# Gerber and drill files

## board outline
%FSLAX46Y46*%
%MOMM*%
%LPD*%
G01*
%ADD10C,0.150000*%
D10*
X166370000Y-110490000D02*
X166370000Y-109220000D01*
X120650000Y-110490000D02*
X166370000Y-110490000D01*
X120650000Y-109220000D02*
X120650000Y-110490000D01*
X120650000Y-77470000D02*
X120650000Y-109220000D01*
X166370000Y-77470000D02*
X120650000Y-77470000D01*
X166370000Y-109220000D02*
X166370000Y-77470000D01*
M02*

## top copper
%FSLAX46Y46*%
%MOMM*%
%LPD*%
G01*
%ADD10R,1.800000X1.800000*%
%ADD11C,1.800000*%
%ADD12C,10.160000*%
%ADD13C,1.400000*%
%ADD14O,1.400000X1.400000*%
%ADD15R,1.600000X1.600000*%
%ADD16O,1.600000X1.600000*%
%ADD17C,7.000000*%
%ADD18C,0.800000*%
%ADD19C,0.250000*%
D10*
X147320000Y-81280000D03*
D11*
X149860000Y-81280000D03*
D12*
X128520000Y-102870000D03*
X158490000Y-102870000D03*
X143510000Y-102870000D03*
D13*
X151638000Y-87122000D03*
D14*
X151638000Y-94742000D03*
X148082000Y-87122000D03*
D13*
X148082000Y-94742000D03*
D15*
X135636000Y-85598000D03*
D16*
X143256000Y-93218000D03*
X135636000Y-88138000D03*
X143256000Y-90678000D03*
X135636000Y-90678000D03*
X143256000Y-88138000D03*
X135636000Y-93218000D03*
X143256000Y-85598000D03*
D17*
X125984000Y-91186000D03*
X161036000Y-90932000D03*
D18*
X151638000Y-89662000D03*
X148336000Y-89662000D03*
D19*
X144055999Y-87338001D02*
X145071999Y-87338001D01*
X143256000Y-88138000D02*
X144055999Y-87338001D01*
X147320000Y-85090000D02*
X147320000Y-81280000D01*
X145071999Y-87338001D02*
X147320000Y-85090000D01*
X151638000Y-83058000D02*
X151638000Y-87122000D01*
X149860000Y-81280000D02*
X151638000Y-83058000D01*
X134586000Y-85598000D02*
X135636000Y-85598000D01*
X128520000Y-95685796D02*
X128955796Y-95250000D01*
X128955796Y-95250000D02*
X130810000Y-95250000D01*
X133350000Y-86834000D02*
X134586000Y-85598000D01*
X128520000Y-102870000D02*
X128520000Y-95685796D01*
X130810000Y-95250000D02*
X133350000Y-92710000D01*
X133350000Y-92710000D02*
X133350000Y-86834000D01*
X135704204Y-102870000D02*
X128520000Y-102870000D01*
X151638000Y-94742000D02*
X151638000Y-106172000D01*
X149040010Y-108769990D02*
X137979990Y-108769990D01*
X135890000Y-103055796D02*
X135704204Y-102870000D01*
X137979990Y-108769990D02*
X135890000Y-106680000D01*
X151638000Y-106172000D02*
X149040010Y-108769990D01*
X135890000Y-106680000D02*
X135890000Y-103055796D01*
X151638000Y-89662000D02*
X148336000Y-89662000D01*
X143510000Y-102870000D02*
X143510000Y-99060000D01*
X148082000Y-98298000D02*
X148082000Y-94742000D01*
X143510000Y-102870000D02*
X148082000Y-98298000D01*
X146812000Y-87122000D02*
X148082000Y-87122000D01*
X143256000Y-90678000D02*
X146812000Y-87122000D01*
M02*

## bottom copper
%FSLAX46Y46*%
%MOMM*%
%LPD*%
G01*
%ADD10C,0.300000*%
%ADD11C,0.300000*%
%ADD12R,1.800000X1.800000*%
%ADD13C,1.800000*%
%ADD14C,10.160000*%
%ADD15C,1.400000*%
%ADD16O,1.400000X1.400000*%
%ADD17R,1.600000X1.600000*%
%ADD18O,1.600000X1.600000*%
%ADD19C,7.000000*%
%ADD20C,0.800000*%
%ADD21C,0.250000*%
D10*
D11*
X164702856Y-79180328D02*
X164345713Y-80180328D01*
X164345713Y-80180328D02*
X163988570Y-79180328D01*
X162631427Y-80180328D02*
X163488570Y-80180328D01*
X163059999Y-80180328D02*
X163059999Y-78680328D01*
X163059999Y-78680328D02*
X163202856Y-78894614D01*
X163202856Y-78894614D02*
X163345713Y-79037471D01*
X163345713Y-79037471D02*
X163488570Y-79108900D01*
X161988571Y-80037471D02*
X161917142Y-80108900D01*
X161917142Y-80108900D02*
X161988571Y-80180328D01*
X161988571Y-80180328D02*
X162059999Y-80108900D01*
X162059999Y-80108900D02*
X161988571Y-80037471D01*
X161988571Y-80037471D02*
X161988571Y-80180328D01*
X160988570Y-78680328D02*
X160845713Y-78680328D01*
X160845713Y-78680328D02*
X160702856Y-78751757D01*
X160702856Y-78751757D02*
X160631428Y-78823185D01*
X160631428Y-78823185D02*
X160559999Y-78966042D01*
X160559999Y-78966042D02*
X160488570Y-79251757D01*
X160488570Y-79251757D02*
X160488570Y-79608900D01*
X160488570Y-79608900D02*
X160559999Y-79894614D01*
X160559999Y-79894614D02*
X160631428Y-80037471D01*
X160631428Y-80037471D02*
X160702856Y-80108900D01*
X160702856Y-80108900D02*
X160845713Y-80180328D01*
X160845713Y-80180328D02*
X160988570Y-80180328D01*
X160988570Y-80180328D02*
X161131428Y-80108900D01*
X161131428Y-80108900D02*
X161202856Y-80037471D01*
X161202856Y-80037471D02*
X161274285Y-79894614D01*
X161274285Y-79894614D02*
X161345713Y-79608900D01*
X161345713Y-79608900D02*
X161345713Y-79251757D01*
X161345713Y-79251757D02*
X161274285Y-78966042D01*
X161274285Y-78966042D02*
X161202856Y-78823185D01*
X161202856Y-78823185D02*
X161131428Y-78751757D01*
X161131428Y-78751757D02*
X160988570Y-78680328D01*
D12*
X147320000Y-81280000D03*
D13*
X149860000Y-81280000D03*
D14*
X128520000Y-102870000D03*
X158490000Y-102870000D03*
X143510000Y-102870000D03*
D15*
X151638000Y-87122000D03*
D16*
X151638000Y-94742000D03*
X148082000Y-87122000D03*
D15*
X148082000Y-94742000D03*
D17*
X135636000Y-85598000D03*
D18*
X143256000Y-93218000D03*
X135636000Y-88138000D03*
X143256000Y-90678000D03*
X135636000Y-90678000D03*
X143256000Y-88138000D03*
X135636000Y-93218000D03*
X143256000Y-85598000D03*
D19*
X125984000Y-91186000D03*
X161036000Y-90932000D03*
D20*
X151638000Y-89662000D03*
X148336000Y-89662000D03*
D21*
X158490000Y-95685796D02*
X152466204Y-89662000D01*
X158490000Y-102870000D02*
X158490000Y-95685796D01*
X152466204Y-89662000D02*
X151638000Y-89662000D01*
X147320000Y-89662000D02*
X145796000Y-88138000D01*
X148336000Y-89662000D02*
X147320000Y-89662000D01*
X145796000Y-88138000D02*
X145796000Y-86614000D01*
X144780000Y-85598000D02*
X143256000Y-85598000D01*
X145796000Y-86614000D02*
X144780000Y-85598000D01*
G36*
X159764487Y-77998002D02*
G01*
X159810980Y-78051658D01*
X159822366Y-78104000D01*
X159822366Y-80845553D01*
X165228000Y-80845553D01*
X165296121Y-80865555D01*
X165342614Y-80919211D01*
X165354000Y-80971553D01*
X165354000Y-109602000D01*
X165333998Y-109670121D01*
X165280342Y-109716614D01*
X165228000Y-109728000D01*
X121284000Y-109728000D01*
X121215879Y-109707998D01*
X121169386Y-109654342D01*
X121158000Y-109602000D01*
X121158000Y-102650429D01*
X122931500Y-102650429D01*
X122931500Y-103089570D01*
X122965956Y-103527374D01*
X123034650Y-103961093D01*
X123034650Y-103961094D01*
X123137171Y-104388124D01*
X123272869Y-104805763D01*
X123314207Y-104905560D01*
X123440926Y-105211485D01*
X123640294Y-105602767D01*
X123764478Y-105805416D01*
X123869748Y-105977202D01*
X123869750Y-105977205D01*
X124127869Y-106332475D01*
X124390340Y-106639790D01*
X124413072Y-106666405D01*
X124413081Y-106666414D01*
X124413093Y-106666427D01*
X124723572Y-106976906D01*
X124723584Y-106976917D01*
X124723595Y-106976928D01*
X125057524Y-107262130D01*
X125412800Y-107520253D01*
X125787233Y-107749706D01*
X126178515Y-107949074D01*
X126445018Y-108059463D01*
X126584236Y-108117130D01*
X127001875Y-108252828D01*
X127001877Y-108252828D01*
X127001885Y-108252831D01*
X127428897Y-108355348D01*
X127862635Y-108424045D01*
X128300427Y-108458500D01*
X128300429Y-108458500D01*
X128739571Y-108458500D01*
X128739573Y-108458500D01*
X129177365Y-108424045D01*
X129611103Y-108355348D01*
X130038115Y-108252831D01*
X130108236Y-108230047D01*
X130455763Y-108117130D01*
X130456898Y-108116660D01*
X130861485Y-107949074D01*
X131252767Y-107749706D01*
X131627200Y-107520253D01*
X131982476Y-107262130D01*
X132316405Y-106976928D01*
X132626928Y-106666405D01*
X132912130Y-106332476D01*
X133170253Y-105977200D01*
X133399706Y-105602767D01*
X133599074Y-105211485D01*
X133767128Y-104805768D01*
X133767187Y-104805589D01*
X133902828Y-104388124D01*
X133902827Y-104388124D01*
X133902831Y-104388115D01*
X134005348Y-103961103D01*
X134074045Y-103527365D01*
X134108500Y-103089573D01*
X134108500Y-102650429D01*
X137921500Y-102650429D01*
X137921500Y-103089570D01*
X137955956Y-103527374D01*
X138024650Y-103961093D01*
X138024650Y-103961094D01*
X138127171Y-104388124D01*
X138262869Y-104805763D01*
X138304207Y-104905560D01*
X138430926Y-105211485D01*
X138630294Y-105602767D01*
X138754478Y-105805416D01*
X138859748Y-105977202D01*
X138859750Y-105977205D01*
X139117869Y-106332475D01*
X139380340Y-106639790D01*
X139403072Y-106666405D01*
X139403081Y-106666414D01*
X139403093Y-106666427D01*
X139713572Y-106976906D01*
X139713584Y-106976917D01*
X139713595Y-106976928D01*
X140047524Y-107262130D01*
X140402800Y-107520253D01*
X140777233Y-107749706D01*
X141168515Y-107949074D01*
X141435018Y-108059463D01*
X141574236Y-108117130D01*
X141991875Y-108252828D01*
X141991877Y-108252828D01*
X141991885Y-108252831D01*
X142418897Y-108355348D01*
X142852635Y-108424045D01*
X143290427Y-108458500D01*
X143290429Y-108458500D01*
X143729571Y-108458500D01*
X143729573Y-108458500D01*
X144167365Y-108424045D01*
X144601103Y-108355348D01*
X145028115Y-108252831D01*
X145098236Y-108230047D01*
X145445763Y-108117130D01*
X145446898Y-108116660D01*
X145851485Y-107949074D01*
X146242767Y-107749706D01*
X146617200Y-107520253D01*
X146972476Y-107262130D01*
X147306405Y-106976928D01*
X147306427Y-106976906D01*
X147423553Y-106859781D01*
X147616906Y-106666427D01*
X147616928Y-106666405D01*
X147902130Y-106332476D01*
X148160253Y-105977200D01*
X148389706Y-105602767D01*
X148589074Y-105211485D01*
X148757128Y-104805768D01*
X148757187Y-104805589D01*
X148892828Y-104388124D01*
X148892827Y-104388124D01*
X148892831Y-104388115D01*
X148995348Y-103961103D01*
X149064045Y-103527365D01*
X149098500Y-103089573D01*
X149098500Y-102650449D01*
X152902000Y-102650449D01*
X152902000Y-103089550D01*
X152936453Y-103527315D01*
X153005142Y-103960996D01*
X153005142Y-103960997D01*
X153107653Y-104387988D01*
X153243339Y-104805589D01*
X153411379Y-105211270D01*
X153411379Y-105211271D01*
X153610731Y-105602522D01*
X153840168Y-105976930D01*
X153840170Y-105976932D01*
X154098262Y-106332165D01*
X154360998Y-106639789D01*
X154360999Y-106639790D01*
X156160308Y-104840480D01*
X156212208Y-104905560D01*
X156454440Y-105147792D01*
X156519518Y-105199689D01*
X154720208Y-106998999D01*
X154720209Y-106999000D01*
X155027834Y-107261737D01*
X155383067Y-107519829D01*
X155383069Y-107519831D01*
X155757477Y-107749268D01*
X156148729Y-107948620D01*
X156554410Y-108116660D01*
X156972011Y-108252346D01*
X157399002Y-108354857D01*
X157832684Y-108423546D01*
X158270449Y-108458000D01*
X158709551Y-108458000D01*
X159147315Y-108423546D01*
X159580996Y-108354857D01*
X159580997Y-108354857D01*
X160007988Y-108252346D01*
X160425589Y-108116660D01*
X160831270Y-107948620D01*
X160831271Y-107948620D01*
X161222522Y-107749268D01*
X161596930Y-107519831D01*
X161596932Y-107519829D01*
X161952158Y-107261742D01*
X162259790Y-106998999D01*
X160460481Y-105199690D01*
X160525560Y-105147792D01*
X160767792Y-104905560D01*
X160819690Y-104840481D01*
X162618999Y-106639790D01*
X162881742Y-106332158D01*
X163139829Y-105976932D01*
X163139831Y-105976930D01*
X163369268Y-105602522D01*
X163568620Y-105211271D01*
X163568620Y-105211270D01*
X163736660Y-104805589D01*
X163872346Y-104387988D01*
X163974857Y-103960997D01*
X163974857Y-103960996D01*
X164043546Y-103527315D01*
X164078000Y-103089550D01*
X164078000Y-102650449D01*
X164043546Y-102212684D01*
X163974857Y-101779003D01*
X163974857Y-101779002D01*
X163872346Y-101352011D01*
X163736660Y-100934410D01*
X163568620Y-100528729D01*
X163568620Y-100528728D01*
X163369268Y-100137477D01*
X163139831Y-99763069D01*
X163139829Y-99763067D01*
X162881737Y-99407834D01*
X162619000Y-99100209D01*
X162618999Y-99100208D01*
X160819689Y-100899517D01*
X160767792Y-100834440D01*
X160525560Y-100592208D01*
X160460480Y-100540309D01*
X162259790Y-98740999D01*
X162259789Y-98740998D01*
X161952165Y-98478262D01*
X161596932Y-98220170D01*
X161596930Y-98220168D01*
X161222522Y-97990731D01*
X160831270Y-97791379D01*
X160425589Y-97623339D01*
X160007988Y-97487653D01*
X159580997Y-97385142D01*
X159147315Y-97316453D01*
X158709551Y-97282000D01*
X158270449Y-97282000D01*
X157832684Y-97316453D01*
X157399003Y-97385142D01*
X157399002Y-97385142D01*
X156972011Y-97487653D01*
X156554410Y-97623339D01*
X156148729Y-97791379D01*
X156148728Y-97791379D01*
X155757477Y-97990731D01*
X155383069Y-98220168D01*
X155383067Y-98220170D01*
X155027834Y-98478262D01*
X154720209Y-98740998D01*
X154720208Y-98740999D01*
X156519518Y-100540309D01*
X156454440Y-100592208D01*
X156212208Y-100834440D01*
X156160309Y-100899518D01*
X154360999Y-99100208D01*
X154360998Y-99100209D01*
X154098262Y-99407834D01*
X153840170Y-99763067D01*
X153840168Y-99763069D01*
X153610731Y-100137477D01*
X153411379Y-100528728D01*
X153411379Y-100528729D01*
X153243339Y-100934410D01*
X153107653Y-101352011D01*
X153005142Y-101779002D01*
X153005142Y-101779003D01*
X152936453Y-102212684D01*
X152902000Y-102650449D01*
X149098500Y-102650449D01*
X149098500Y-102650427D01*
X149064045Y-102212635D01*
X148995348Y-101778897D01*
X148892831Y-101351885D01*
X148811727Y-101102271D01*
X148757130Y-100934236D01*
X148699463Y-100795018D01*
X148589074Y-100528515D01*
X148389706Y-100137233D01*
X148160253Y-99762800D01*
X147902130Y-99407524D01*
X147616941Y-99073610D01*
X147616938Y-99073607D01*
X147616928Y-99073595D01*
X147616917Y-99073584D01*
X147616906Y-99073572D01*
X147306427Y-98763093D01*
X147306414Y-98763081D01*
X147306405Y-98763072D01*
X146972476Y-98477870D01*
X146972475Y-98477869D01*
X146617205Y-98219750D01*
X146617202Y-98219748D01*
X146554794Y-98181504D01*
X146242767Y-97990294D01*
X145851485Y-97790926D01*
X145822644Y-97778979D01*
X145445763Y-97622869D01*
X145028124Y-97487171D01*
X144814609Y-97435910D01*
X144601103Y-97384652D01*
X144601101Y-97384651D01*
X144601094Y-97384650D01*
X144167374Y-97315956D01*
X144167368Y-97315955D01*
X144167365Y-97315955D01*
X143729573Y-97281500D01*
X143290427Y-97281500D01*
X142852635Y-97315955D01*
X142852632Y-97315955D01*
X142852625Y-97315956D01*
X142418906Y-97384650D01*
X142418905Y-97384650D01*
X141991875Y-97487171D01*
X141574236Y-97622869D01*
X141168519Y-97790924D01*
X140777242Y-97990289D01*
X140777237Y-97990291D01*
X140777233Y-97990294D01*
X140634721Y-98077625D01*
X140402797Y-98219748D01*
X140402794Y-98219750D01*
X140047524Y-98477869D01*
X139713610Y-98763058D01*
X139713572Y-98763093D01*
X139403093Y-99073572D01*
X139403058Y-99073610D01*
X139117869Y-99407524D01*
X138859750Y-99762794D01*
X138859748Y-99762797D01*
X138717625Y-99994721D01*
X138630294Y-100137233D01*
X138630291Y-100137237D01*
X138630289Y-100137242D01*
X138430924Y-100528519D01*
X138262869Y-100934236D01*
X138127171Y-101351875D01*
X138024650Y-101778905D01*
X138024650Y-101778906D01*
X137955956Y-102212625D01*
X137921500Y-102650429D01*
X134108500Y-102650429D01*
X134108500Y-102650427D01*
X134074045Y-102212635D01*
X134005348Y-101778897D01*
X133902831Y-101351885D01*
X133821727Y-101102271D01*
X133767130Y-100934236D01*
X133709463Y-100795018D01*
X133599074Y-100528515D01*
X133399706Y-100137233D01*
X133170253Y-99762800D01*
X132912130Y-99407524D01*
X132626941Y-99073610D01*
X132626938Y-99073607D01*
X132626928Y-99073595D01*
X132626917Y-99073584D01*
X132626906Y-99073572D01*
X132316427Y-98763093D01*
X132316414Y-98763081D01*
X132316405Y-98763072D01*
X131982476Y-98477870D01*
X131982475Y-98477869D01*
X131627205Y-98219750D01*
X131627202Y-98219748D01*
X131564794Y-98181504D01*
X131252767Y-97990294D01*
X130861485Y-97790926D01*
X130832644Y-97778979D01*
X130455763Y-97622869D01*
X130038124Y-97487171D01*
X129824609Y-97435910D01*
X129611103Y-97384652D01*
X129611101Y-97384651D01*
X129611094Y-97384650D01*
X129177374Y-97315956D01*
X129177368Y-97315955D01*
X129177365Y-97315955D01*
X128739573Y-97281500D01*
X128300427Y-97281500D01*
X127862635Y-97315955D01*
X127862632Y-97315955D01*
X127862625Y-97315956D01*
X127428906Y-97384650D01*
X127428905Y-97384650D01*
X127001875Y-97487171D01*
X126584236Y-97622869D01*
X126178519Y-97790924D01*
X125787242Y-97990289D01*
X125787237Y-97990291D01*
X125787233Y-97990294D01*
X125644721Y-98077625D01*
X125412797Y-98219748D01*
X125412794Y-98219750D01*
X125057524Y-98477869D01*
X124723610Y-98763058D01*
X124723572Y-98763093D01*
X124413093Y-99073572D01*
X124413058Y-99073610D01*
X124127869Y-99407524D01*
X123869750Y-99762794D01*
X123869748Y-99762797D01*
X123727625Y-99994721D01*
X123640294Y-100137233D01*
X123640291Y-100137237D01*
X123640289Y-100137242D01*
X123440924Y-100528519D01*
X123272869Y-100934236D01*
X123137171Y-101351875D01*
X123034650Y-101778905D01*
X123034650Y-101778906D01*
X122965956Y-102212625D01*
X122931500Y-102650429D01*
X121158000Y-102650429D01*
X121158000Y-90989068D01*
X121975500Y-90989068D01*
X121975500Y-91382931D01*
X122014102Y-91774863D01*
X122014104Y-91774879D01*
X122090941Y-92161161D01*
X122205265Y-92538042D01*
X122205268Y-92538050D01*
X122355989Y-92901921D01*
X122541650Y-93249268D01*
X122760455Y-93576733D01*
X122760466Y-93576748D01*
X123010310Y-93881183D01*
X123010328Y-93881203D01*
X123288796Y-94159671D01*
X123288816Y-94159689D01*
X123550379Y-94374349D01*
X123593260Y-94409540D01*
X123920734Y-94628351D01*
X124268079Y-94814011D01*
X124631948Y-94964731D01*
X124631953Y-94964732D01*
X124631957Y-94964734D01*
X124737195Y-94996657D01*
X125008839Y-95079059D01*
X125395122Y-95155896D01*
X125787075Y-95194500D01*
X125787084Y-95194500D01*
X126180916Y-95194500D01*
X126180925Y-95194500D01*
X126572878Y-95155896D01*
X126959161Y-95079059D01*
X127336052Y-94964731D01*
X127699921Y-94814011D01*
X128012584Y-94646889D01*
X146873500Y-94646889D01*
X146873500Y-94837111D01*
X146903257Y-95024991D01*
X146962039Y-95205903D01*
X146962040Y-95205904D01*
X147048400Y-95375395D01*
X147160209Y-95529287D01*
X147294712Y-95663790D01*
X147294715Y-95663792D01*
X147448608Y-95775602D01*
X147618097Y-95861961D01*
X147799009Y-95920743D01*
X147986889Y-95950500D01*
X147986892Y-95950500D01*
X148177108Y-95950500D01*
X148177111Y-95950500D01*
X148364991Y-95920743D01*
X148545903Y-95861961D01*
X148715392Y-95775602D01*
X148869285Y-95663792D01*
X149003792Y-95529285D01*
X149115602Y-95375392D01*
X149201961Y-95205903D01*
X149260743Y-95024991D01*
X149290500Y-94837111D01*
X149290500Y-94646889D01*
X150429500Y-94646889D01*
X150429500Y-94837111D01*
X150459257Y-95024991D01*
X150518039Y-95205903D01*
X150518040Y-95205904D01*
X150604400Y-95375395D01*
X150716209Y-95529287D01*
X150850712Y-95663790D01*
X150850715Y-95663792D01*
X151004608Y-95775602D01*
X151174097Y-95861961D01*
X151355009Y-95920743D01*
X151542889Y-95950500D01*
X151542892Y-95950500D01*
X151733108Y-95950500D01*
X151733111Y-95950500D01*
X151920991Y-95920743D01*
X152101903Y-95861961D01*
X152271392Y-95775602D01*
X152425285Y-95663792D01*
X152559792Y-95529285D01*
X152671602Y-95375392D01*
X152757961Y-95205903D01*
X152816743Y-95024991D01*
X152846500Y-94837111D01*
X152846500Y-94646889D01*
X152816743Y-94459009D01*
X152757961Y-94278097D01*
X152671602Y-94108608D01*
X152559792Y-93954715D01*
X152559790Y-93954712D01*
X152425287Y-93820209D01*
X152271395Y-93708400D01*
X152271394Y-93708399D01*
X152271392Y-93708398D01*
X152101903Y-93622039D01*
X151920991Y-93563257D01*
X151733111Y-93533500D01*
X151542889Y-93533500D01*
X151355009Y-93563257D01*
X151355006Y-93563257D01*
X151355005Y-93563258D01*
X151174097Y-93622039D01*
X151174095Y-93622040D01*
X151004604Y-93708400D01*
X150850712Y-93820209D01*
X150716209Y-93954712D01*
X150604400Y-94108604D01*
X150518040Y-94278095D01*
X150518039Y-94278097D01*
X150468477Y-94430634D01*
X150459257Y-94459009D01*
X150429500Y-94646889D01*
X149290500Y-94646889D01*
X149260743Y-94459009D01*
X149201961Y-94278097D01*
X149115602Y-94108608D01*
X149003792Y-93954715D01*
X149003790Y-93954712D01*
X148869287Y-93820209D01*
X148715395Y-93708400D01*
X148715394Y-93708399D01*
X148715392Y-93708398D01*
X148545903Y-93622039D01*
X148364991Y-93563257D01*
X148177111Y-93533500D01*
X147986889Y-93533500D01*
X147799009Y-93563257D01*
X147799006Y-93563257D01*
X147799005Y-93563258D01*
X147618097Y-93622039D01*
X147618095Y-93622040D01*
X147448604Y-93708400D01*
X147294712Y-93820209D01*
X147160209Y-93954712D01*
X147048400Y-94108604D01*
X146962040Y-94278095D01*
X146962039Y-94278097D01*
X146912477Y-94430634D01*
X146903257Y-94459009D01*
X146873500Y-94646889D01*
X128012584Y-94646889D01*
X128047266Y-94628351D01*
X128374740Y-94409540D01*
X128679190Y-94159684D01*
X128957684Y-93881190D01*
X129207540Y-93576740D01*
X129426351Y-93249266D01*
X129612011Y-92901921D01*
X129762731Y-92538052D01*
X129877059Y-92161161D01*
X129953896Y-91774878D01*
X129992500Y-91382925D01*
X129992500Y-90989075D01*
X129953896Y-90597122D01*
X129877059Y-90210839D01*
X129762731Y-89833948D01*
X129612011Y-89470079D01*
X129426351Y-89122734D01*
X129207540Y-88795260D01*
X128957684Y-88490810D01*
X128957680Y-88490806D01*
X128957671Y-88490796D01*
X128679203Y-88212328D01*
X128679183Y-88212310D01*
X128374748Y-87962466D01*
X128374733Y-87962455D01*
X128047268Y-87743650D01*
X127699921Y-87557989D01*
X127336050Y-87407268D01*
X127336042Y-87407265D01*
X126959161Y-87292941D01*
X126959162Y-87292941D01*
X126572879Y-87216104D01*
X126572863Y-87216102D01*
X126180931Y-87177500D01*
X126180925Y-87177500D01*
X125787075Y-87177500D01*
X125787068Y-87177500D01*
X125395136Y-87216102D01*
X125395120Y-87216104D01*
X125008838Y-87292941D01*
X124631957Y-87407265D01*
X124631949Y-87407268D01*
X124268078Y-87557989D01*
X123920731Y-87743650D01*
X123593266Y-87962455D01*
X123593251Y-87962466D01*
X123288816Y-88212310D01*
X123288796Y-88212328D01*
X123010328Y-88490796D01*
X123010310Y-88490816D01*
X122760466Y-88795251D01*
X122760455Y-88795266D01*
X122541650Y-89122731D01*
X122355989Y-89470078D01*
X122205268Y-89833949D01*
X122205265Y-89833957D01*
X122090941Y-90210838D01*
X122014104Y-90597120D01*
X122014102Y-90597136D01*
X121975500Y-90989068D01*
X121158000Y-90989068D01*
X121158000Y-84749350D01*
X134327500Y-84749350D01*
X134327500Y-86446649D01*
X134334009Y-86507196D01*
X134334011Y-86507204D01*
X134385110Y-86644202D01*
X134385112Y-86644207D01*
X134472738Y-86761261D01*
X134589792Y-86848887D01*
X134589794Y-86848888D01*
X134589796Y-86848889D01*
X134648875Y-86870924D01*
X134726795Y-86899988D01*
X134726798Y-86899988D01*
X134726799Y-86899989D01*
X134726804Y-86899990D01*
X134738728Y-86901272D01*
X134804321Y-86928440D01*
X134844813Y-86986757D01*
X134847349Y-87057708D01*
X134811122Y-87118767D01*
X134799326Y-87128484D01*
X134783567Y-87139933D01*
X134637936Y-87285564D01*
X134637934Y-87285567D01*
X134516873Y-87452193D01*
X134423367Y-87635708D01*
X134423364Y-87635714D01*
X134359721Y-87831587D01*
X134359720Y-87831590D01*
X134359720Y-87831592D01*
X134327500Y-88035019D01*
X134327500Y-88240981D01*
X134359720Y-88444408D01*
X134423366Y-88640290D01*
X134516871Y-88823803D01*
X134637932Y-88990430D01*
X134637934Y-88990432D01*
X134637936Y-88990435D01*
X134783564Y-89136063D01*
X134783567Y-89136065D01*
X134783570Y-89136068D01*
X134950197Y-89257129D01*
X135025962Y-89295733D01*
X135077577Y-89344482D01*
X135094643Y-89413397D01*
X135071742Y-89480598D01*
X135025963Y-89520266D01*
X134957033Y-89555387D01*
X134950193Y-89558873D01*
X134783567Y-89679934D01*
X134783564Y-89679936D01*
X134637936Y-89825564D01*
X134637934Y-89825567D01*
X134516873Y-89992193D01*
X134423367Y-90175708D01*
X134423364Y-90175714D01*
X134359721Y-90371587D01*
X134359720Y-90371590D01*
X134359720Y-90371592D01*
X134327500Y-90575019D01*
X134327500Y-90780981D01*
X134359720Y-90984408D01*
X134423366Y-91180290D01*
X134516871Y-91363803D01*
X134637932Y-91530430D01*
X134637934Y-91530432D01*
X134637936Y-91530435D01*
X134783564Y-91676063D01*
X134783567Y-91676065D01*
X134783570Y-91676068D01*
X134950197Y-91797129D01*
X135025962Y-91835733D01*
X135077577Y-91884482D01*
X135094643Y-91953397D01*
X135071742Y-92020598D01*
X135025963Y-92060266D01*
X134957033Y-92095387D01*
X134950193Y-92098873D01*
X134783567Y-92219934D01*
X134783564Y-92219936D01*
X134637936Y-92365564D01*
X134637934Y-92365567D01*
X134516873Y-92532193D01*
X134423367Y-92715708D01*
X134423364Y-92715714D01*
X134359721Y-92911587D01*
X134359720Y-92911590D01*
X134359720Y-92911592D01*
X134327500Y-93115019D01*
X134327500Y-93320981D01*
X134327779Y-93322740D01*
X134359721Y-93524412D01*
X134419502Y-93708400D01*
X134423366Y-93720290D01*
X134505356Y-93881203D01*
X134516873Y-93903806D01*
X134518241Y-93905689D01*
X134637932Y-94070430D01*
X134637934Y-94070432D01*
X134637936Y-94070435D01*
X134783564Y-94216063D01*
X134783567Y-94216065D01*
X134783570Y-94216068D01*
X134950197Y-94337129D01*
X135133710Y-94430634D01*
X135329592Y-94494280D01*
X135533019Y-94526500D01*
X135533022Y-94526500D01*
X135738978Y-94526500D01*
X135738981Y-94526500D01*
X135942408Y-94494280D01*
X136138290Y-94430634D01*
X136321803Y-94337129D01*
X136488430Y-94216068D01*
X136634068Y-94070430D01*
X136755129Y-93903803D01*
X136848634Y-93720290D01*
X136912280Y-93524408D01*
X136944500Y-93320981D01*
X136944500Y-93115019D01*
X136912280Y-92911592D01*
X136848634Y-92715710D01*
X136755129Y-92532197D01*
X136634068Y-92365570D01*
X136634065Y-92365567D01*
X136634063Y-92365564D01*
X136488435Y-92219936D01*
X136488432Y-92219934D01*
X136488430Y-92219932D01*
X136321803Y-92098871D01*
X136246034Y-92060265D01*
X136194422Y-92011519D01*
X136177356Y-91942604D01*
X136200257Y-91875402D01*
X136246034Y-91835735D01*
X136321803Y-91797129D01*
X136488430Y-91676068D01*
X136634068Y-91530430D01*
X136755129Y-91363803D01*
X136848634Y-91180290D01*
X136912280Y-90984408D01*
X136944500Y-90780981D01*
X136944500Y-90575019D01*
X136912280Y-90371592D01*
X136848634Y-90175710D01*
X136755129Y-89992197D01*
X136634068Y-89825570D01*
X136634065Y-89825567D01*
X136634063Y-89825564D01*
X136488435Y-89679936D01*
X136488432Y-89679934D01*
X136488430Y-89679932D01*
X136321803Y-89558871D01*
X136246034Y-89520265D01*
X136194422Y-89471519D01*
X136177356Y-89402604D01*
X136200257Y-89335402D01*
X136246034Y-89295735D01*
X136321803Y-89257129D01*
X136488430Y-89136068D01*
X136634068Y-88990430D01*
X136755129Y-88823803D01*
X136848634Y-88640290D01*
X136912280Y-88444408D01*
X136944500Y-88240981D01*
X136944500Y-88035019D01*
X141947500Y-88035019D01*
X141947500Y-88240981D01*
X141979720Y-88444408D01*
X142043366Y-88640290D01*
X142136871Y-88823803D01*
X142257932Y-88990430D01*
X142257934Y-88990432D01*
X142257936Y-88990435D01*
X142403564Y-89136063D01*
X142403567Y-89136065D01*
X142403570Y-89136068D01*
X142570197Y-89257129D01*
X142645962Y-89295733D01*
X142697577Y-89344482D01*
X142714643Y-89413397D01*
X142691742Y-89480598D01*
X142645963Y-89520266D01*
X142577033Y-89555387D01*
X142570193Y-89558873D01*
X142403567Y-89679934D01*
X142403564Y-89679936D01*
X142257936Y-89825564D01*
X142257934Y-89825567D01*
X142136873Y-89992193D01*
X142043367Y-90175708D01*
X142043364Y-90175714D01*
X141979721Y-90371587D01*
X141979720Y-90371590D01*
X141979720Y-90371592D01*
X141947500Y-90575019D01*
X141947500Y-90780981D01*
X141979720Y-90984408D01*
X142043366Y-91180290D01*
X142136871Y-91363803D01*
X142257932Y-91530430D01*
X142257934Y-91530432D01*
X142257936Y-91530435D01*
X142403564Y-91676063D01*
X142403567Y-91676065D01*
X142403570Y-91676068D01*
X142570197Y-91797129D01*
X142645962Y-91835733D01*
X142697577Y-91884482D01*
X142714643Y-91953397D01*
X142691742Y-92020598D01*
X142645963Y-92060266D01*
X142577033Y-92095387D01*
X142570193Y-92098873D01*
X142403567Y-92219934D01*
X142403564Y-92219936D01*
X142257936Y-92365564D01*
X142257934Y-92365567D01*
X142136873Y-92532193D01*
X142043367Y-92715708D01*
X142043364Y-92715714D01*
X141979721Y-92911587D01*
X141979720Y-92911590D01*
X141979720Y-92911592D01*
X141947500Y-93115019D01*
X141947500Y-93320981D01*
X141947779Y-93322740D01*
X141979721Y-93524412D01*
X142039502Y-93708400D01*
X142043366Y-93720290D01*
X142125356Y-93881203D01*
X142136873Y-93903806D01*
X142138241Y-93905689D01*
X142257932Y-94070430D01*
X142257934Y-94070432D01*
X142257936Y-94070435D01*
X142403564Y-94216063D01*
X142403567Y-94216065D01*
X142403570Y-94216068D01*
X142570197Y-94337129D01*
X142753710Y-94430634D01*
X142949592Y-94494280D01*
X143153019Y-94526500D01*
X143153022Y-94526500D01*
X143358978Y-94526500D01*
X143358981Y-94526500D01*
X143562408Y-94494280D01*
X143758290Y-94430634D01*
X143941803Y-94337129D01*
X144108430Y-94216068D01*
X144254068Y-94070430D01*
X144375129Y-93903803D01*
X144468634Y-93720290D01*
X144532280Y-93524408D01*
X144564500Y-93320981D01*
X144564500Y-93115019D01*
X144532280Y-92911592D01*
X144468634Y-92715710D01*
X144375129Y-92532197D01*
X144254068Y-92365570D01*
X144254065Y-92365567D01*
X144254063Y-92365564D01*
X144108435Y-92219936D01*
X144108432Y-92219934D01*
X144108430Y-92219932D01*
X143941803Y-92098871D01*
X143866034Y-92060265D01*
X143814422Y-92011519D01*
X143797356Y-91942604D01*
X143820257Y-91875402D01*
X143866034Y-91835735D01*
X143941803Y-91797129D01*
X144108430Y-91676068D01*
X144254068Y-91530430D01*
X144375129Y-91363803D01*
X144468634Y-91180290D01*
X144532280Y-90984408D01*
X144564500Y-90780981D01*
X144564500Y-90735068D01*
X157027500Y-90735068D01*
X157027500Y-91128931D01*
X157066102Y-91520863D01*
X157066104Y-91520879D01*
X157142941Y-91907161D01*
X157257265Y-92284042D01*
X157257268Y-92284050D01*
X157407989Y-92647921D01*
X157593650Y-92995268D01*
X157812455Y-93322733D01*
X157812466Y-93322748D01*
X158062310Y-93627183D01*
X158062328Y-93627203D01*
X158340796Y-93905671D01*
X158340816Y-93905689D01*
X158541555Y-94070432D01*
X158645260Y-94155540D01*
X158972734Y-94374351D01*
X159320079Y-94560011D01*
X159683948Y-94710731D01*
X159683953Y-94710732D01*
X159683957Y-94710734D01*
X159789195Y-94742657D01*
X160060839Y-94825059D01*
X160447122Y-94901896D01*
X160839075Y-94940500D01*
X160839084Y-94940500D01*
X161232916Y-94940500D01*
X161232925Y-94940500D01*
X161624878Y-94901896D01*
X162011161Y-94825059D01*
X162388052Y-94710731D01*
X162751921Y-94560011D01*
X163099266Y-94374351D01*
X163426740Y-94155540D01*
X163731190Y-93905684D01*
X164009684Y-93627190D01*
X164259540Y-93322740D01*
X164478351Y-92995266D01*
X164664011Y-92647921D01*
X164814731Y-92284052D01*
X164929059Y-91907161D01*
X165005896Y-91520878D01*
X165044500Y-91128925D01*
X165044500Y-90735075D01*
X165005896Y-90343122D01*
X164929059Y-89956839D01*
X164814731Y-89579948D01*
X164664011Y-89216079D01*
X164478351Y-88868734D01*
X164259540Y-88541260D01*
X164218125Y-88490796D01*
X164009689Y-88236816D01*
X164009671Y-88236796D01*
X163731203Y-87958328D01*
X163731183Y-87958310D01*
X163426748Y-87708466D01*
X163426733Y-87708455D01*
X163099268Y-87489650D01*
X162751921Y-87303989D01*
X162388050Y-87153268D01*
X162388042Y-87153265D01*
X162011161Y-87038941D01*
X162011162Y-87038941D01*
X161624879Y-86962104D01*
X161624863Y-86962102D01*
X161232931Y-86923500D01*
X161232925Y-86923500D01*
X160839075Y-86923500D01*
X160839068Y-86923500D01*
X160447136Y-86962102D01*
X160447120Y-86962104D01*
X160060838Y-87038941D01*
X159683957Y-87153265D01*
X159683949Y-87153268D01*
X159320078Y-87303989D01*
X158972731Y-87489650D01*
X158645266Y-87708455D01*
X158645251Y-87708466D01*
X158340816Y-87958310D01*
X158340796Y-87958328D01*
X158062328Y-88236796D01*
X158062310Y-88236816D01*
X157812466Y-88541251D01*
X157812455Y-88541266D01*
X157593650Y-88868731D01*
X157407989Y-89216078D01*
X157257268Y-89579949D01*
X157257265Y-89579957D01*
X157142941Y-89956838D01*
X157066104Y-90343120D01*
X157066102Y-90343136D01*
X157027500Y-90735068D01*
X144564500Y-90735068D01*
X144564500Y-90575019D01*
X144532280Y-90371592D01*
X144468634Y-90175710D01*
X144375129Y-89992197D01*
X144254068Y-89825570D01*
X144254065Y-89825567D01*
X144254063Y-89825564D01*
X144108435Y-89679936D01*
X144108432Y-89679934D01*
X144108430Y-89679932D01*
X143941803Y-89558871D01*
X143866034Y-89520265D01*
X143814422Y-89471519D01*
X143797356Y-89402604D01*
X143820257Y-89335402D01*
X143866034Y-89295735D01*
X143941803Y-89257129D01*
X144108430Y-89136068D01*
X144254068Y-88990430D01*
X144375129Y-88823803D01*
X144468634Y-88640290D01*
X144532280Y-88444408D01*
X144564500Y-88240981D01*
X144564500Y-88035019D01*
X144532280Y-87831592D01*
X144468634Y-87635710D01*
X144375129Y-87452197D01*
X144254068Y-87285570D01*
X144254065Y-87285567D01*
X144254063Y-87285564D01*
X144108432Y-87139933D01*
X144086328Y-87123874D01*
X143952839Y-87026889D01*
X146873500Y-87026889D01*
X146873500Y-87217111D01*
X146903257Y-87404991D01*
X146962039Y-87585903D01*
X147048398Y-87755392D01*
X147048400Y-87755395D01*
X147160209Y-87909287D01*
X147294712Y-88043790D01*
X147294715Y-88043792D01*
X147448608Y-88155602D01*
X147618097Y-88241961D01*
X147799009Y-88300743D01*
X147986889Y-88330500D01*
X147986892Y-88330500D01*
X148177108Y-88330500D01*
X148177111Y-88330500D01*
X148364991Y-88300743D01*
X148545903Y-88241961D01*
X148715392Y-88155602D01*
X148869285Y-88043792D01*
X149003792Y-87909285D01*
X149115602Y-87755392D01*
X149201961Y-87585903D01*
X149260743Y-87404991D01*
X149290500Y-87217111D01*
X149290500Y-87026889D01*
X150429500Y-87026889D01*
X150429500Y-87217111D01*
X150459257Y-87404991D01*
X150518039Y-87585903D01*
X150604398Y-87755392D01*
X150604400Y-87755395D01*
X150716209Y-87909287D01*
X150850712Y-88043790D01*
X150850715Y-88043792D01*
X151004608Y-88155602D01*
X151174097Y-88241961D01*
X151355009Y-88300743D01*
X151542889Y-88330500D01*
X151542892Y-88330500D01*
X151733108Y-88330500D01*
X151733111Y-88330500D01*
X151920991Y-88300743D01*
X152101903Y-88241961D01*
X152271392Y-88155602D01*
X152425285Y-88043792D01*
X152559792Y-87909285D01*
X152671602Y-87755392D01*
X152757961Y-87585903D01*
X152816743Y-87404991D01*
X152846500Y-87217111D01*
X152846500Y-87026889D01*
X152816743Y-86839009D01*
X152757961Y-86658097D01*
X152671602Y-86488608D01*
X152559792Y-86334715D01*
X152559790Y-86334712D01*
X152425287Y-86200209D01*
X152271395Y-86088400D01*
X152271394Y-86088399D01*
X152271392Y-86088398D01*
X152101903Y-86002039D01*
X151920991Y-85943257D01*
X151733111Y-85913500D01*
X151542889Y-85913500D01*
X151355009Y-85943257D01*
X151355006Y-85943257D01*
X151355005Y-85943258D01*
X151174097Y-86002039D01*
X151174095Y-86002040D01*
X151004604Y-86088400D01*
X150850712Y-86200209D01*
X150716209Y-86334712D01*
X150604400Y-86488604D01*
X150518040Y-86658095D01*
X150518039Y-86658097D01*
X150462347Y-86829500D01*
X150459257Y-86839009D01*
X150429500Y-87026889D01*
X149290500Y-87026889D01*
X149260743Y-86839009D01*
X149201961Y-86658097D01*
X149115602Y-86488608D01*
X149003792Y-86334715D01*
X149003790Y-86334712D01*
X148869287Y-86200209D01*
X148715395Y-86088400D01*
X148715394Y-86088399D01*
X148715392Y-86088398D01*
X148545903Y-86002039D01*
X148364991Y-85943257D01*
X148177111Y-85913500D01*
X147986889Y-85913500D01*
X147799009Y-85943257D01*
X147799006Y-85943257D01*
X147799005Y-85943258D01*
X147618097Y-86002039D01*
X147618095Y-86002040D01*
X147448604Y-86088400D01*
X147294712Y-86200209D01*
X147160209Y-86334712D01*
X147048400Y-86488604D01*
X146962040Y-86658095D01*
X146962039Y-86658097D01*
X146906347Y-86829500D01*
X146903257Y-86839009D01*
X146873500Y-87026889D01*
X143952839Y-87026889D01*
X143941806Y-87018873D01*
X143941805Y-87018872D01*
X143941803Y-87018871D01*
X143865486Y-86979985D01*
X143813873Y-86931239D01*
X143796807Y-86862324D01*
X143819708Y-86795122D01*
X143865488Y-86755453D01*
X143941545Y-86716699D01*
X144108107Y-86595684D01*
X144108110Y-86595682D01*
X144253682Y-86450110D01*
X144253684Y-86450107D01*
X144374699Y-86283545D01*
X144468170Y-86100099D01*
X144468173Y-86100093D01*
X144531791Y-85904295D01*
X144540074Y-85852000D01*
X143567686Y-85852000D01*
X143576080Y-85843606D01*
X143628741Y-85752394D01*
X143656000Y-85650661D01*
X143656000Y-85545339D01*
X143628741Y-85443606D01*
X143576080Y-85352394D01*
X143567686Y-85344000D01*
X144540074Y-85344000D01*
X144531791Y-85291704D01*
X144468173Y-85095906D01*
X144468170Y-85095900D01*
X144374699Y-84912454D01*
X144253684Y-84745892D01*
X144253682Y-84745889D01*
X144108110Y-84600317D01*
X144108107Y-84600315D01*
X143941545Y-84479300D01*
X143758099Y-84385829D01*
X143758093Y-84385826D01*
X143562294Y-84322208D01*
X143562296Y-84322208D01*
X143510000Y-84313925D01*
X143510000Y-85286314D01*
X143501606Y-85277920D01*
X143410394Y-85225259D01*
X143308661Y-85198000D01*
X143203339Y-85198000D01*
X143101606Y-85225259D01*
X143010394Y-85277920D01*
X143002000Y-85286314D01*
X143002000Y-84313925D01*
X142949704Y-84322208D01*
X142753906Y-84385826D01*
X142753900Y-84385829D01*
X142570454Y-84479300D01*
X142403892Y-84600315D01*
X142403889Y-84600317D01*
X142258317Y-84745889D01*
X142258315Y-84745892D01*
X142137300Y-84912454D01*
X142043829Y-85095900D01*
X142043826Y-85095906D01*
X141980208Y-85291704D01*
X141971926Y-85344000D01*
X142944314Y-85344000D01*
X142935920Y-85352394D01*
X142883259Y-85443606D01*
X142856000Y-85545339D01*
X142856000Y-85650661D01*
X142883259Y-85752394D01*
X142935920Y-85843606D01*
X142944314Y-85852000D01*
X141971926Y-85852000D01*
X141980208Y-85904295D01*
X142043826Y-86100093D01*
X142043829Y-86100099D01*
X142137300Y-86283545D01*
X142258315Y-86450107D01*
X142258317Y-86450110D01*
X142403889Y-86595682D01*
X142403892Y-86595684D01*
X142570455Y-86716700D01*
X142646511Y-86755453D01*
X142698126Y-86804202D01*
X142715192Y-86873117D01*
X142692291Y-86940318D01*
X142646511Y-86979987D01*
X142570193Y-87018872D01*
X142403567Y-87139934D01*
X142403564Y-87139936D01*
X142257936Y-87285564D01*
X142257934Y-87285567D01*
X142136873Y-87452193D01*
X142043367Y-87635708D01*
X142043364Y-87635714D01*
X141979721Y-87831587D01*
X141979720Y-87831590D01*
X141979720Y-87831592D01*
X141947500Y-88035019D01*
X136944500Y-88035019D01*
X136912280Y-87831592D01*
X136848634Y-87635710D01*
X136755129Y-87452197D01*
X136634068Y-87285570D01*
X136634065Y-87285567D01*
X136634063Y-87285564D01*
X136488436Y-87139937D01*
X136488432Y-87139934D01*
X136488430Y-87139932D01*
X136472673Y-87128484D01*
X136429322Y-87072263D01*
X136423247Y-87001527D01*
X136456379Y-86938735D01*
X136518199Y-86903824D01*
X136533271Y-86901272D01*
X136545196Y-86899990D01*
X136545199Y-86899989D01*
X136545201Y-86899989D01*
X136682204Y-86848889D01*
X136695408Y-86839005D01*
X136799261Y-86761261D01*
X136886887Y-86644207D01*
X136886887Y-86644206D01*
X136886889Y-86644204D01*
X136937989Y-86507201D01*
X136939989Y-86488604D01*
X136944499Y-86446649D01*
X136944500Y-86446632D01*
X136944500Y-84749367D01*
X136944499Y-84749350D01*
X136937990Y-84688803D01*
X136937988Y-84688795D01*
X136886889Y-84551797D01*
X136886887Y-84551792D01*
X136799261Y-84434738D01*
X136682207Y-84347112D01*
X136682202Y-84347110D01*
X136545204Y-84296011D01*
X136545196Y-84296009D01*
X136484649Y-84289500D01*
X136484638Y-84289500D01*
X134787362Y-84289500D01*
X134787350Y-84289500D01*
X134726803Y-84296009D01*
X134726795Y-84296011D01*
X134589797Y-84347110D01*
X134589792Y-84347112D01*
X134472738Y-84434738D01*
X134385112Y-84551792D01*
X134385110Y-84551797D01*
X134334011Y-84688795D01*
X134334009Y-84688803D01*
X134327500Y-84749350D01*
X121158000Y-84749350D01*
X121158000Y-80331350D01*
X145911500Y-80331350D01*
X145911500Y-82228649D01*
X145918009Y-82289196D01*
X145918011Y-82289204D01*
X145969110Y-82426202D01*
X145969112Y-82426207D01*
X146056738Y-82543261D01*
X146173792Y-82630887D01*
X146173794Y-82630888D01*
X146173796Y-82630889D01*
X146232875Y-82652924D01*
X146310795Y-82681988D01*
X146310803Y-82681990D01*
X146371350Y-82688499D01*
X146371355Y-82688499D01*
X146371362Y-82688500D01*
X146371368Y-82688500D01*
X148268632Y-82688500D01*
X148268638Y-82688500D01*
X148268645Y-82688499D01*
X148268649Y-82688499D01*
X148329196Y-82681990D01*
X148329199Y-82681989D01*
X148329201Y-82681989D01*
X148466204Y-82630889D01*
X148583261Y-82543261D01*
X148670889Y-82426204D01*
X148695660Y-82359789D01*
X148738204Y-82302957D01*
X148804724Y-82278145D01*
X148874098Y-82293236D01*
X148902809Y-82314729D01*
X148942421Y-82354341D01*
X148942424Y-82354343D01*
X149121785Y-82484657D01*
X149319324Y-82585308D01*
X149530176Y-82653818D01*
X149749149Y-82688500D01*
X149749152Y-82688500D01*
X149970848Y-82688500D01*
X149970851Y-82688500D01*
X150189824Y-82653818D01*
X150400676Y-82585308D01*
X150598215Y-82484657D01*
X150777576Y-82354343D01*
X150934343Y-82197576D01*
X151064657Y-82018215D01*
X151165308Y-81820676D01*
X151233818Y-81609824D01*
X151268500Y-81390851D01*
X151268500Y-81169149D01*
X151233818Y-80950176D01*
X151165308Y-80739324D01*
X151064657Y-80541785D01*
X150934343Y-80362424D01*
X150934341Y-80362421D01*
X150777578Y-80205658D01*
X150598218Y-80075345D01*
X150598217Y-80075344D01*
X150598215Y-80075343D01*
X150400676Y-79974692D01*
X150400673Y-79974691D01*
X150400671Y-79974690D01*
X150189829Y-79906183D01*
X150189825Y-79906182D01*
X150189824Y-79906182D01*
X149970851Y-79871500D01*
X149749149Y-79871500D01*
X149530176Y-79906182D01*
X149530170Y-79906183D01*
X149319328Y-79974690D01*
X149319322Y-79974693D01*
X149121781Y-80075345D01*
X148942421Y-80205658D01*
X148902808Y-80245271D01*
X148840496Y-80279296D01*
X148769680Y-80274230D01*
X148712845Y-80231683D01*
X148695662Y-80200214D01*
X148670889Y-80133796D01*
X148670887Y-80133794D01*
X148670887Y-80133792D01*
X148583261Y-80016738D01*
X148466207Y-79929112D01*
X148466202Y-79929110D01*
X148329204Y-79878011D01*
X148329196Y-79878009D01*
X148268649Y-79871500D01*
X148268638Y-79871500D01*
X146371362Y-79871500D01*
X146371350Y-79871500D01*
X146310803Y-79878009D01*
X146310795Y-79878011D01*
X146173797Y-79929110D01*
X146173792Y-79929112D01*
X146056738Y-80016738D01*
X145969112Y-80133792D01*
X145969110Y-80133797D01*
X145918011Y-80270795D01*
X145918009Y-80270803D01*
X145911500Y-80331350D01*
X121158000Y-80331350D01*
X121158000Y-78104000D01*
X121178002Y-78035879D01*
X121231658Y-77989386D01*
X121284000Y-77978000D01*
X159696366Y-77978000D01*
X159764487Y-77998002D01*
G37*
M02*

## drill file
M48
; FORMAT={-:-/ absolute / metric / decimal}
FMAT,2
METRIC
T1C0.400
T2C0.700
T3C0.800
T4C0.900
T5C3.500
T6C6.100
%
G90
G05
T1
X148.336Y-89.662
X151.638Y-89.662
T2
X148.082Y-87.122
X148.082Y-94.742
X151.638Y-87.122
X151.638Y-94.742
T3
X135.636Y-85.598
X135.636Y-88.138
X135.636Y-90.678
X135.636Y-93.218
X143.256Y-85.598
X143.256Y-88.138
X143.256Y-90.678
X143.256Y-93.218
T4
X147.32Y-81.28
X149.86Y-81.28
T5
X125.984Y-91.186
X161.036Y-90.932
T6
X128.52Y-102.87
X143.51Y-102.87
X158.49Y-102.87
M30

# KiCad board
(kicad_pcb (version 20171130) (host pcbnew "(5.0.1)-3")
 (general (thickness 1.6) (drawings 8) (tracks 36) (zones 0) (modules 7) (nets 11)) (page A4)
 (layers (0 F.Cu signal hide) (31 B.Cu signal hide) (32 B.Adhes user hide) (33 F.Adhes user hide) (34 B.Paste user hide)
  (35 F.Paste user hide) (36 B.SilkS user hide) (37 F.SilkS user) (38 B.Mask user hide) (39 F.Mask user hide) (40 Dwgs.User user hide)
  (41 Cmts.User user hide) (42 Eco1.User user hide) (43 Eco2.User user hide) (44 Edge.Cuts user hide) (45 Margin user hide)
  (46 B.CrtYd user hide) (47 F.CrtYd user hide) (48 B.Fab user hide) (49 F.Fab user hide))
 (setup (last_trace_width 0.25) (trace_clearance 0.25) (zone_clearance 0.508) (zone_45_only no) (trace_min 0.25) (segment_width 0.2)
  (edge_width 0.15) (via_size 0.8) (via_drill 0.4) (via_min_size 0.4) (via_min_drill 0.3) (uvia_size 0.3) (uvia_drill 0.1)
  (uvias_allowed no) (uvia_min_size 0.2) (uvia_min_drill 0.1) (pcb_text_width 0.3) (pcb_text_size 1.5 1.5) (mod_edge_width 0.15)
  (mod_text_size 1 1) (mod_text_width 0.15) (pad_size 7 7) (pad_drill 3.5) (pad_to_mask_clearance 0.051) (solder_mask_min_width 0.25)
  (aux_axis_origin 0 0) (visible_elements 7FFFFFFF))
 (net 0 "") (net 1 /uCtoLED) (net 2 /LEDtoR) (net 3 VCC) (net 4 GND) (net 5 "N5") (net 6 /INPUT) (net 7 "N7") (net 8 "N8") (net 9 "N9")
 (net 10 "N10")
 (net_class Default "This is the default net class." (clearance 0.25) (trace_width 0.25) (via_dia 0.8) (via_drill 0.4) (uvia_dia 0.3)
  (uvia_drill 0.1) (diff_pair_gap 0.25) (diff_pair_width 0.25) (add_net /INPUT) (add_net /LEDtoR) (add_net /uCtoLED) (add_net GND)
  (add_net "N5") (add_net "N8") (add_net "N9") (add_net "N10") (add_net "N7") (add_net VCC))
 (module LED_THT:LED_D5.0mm (layer F.Cu) (at 147.32 81.28)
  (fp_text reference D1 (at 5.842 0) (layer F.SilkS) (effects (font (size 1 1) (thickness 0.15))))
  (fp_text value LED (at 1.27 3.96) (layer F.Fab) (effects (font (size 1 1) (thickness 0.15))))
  (pad 1 thru_hole rect (at 0 0) (size 1.8 1.8) (drill 0.9) (layers *.Cu *.Mask) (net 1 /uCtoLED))
  (pad 2 thru_hole circle (at 2.54 0) (size 1.8 1.8) (drill 0.9) (layers *.Cu *.Mask) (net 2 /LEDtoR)))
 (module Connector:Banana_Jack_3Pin (layer F.Cu) (at 128.52 102.87)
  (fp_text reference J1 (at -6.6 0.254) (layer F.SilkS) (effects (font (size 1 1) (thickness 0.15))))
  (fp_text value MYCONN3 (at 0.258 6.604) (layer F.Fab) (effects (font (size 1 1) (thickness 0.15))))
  (pad 1 thru_hole circle (at 0 0) (size 10.16 10.16) (drill 6.1) (layers *.Cu *.Mask) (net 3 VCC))
  (pad 3 thru_hole circle (at 29.97 0) (size 10.16 10.16) (drill 6.1) (layers *.Cu *.Mask) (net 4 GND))
  (pad 2 thru_hole circle (at 14.99 0) (size 10.16 10.16) (drill 6.1) (layers *.Cu *.Mask) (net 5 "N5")))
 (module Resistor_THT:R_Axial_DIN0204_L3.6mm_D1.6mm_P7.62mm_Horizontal (layer F.Cu) (at 151.638 87.122 270)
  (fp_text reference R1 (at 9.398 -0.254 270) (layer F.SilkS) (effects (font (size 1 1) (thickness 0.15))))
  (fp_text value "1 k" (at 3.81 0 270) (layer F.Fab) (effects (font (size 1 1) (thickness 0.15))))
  (pad 1 thru_hole circle (at 0 0 270) (size 1.4 1.4) (drill 0.7) (layers *.Cu *.Mask) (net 2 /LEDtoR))
  (pad 2 thru_hole oval (at 7.62 0 270) (size 1.4 1.4) (drill 0.7) (layers *.Cu *.Mask) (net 3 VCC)))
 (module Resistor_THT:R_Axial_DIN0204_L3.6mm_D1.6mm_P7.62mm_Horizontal (layer F.Cu) (at 148.082 94.742 90)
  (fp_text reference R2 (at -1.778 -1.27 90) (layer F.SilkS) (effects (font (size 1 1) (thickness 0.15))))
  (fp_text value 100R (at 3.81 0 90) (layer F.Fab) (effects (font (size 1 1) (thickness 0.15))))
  (pad 2 thru_hole oval (at 7.62 0 90) (size 1.4 1.4) (drill 0.7) (layers *.Cu *.Mask) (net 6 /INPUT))
  (pad 1 thru_hole circle (at 0 0 90) (size 1.4 1.4) (drill 0.7) (layers *.Cu *.Mask) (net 5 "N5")))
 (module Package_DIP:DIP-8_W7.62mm (layer F.Cu) (at 135.636 85.598)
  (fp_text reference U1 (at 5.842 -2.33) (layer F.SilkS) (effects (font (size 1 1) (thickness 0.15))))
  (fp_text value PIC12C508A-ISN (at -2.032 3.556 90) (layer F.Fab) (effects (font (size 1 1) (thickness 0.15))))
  (pad 1 thru_hole rect (at 0 0) (size 1.6 1.6) (drill 0.8) (layers *.Cu *.Mask) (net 3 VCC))
  (pad 5 thru_hole oval (at 7.62 7.62) (size 1.6 1.6) (drill 0.8) (layers *.Cu *.Mask) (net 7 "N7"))
  (pad 2 thru_hole oval (at 0 2.54) (size 1.6 1.6) (drill 0.8) (layers *.Cu *.Mask) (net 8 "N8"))
  (pad 6 thru_hole oval (at 7.62 5.08) (size 1.6 1.6) (drill 0.8) (layers *.Cu *.Mask) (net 6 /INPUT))
  (pad 3 thru_hole oval (at 0 5.08) (size 1.6 1.6) (drill 0.8) (layers *.Cu *.Mask) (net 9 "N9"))
  (pad 7 thru_hole oval (at 7.62 2.54) (size 1.6 1.6) (drill 0.8) (layers *.Cu *.Mask) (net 1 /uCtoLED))
  (pad 4 thru_hole oval (at 0 7.62) (size 1.6 1.6) (drill 0.8) (layers *.Cu *.Mask) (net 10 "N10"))
  (pad 8 thru_hole oval (at 7.62 0) (size 1.6 1.6) (drill 0.8) (layers *.Cu *.Mask) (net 4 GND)))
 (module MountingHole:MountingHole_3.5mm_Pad (layer F.Cu) (at 125.984 91.186)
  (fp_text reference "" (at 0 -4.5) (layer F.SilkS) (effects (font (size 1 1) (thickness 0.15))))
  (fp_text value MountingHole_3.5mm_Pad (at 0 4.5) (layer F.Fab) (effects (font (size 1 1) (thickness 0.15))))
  (pad 1 thru_hole circle (at 0 0) (size 7 7) (drill 3.5) (layers *.Cu *.Mask)))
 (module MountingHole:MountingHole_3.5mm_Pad (layer F.Cu) (at 161.036 90.932)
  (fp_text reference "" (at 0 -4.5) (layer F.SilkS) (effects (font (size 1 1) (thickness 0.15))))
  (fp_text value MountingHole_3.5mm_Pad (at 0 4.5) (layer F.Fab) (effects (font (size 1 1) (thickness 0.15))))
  (pad 2 thru_hole circle (at 0 0) (size 7 7) (drill 3.5) (layers *.Cu *.Mask Dwgs.User)))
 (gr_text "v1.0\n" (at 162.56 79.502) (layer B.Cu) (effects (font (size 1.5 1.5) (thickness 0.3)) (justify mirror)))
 (gr_line (start 166.37 110.49) (end 166.37 109.22) (layer Edge.Cuts) (width 0.15))
 (gr_line (start 120.65 110.49) (end 166.37 110.49) (layer Edge.Cuts) (width 0.15))
 (gr_line (start 120.65 109.22) (end 120.65 110.49) (layer Edge.Cuts) (width 0.15))
 (gr_line (start 120.65 77.47) (end 120.65 109.22) (layer Edge.Cuts) (width 0.15))
 (gr_line (start 166.37 77.47) (end 120.65 77.47) (layer Edge.Cuts) (width 0.15))
 (gr_line (start 166.37 109.22) (end 166.37 77.47) (layer Edge.Cuts) (width 0.15))
 (segment (start 144.055999 87.338001) (end 145.071999 87.338001) (width 0.25) (layer F.Cu) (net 1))
 (segment (start 143.256 88.138) (end 144.055999 87.338001) (width 0.25) (layer F.Cu) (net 1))
 (segment (start 147.32 85.09) (end 147.32 81.28) (width 0.25) (layer F.Cu) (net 1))
 (segment (start 145.071999 87.338001) (end 147.32 85.09) (width 0.25) (layer F.Cu) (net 1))
 (segment (start 151.638 83.058) (end 151.638 87.122) (width 0.25) (layer F.Cu) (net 2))
 (segment (start 149.86 81.28) (end 151.638 83.058) (width 0.25) (layer F.Cu) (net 2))
 (segment (start 134.586 85.598) (end 135.636 85.598) (width 0.25) (layer F.Cu) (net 3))
 (segment (start 128.52 95.685796) (end 128.955796 95.25) (width 0.25) (layer F.Cu) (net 3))
 (segment (start 128.955796 95.25) (end 130.81 95.25) (width 0.25) (layer F.Cu) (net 3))
 (segment (start 133.35 86.834) (end 134.586 85.598) (width 0.25) (layer F.Cu) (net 3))
 (segment (start 128.52 102.87) (end 128.52 95.685796) (width 0.25) (layer F.Cu) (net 3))
 (segment (start 130.81 95.25) (end 133.35 92.71) (width 0.25) (layer F.Cu) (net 3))
 (segment (start 133.35 92.71) (end 133.35 86.834) (width 0.25) (layer F.Cu) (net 3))
 (segment (start 135.704204 102.87) (end 128.52 102.87) (width 0.25) (layer F.Cu) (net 3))
 (segment (start 151.638 94.742) (end 151.638 106.172) (width 0.25) (layer F.Cu) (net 3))
 (segment (start 149.04001 108.76999) (end 137.97999 108.76999) (width 0.25) (layer F.Cu) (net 3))
 (segment (start 135.89 103.055796) (end 135.704204 102.87) (width 0.25) (layer F.Cu) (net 3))
 (segment (start 137.97999 108.76999) (end 135.89 106.68) (width 0.25) (layer F.Cu) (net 3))
 (segment (start 151.638 106.172) (end 149.04001 108.76999) (width 0.25) (layer F.Cu) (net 3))
 (segment (start 135.89 106.68) (end 135.89 103.055796) (width 0.25) (layer F.Cu) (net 3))
 (segment (start 158.49 95.685796) (end 152.466204 89.662) (width 0.25) (layer B.Cu) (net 4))
 (segment (start 158.49 102.87) (end 158.49 95.685796) (width 0.25) (layer B.Cu) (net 4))
 (via (at 151.638 89.662) (size 0.8) (drill 0.4) (layers F.Cu B.Cu) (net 4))
 (segment (start 152.466204 89.662) (end 151.638 89.662) (width 0.25) (layer B.Cu) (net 4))
 (segment (start 151.638 89.662) (end 148.336 89.662) (width 0.25) (layer F.Cu) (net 4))
 (via (at 148.336 89.662) (size 0.8) (drill 0.4) (layers F.Cu B.Cu) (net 4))
 (segment (start 147.32 89.662) (end 145.796 88.138) (width 0.25) (layer B.Cu) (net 4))
 (segment (start 148.336 89.662) (end 147.32 89.662) (width 0.25) (layer B.Cu) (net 4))
 (segment (start 145.796 88.138) (end 145.796 86.614) (width 0.25) (layer B.Cu) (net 4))
 (segment (start 144.78 85.598) (end 143.256 85.598) (width 0.25) (layer B.Cu) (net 4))
 (segment (start 145.796 86.614) (end 144.78 85.598) (width 0.25) (layer B.Cu) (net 4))
 (segment (start 143.51 102.87) (end 143.51 99.06) (width 0.25) (layer F.Cu) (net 5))
 (segment (start 148.082 98.298) (end 148.082 94.742) (width 0.25) (layer F.Cu) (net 5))
 (segment (start 143.51 102.87) (end 148.082 98.298) (width 0.25) (layer F.Cu) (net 5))
 (segment (start 146.812 87.122) (end 148.082 87.122) (width 0.25) (layer F.Cu) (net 6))
 (segment (start 143.256 90.678) (end 146.812 87.122) (width 0.25) (layer F.Cu) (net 6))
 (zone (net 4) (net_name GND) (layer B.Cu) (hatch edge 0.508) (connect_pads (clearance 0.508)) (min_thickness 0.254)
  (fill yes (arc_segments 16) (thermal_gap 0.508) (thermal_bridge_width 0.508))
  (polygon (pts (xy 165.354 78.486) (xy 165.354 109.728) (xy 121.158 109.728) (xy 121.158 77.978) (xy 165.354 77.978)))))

